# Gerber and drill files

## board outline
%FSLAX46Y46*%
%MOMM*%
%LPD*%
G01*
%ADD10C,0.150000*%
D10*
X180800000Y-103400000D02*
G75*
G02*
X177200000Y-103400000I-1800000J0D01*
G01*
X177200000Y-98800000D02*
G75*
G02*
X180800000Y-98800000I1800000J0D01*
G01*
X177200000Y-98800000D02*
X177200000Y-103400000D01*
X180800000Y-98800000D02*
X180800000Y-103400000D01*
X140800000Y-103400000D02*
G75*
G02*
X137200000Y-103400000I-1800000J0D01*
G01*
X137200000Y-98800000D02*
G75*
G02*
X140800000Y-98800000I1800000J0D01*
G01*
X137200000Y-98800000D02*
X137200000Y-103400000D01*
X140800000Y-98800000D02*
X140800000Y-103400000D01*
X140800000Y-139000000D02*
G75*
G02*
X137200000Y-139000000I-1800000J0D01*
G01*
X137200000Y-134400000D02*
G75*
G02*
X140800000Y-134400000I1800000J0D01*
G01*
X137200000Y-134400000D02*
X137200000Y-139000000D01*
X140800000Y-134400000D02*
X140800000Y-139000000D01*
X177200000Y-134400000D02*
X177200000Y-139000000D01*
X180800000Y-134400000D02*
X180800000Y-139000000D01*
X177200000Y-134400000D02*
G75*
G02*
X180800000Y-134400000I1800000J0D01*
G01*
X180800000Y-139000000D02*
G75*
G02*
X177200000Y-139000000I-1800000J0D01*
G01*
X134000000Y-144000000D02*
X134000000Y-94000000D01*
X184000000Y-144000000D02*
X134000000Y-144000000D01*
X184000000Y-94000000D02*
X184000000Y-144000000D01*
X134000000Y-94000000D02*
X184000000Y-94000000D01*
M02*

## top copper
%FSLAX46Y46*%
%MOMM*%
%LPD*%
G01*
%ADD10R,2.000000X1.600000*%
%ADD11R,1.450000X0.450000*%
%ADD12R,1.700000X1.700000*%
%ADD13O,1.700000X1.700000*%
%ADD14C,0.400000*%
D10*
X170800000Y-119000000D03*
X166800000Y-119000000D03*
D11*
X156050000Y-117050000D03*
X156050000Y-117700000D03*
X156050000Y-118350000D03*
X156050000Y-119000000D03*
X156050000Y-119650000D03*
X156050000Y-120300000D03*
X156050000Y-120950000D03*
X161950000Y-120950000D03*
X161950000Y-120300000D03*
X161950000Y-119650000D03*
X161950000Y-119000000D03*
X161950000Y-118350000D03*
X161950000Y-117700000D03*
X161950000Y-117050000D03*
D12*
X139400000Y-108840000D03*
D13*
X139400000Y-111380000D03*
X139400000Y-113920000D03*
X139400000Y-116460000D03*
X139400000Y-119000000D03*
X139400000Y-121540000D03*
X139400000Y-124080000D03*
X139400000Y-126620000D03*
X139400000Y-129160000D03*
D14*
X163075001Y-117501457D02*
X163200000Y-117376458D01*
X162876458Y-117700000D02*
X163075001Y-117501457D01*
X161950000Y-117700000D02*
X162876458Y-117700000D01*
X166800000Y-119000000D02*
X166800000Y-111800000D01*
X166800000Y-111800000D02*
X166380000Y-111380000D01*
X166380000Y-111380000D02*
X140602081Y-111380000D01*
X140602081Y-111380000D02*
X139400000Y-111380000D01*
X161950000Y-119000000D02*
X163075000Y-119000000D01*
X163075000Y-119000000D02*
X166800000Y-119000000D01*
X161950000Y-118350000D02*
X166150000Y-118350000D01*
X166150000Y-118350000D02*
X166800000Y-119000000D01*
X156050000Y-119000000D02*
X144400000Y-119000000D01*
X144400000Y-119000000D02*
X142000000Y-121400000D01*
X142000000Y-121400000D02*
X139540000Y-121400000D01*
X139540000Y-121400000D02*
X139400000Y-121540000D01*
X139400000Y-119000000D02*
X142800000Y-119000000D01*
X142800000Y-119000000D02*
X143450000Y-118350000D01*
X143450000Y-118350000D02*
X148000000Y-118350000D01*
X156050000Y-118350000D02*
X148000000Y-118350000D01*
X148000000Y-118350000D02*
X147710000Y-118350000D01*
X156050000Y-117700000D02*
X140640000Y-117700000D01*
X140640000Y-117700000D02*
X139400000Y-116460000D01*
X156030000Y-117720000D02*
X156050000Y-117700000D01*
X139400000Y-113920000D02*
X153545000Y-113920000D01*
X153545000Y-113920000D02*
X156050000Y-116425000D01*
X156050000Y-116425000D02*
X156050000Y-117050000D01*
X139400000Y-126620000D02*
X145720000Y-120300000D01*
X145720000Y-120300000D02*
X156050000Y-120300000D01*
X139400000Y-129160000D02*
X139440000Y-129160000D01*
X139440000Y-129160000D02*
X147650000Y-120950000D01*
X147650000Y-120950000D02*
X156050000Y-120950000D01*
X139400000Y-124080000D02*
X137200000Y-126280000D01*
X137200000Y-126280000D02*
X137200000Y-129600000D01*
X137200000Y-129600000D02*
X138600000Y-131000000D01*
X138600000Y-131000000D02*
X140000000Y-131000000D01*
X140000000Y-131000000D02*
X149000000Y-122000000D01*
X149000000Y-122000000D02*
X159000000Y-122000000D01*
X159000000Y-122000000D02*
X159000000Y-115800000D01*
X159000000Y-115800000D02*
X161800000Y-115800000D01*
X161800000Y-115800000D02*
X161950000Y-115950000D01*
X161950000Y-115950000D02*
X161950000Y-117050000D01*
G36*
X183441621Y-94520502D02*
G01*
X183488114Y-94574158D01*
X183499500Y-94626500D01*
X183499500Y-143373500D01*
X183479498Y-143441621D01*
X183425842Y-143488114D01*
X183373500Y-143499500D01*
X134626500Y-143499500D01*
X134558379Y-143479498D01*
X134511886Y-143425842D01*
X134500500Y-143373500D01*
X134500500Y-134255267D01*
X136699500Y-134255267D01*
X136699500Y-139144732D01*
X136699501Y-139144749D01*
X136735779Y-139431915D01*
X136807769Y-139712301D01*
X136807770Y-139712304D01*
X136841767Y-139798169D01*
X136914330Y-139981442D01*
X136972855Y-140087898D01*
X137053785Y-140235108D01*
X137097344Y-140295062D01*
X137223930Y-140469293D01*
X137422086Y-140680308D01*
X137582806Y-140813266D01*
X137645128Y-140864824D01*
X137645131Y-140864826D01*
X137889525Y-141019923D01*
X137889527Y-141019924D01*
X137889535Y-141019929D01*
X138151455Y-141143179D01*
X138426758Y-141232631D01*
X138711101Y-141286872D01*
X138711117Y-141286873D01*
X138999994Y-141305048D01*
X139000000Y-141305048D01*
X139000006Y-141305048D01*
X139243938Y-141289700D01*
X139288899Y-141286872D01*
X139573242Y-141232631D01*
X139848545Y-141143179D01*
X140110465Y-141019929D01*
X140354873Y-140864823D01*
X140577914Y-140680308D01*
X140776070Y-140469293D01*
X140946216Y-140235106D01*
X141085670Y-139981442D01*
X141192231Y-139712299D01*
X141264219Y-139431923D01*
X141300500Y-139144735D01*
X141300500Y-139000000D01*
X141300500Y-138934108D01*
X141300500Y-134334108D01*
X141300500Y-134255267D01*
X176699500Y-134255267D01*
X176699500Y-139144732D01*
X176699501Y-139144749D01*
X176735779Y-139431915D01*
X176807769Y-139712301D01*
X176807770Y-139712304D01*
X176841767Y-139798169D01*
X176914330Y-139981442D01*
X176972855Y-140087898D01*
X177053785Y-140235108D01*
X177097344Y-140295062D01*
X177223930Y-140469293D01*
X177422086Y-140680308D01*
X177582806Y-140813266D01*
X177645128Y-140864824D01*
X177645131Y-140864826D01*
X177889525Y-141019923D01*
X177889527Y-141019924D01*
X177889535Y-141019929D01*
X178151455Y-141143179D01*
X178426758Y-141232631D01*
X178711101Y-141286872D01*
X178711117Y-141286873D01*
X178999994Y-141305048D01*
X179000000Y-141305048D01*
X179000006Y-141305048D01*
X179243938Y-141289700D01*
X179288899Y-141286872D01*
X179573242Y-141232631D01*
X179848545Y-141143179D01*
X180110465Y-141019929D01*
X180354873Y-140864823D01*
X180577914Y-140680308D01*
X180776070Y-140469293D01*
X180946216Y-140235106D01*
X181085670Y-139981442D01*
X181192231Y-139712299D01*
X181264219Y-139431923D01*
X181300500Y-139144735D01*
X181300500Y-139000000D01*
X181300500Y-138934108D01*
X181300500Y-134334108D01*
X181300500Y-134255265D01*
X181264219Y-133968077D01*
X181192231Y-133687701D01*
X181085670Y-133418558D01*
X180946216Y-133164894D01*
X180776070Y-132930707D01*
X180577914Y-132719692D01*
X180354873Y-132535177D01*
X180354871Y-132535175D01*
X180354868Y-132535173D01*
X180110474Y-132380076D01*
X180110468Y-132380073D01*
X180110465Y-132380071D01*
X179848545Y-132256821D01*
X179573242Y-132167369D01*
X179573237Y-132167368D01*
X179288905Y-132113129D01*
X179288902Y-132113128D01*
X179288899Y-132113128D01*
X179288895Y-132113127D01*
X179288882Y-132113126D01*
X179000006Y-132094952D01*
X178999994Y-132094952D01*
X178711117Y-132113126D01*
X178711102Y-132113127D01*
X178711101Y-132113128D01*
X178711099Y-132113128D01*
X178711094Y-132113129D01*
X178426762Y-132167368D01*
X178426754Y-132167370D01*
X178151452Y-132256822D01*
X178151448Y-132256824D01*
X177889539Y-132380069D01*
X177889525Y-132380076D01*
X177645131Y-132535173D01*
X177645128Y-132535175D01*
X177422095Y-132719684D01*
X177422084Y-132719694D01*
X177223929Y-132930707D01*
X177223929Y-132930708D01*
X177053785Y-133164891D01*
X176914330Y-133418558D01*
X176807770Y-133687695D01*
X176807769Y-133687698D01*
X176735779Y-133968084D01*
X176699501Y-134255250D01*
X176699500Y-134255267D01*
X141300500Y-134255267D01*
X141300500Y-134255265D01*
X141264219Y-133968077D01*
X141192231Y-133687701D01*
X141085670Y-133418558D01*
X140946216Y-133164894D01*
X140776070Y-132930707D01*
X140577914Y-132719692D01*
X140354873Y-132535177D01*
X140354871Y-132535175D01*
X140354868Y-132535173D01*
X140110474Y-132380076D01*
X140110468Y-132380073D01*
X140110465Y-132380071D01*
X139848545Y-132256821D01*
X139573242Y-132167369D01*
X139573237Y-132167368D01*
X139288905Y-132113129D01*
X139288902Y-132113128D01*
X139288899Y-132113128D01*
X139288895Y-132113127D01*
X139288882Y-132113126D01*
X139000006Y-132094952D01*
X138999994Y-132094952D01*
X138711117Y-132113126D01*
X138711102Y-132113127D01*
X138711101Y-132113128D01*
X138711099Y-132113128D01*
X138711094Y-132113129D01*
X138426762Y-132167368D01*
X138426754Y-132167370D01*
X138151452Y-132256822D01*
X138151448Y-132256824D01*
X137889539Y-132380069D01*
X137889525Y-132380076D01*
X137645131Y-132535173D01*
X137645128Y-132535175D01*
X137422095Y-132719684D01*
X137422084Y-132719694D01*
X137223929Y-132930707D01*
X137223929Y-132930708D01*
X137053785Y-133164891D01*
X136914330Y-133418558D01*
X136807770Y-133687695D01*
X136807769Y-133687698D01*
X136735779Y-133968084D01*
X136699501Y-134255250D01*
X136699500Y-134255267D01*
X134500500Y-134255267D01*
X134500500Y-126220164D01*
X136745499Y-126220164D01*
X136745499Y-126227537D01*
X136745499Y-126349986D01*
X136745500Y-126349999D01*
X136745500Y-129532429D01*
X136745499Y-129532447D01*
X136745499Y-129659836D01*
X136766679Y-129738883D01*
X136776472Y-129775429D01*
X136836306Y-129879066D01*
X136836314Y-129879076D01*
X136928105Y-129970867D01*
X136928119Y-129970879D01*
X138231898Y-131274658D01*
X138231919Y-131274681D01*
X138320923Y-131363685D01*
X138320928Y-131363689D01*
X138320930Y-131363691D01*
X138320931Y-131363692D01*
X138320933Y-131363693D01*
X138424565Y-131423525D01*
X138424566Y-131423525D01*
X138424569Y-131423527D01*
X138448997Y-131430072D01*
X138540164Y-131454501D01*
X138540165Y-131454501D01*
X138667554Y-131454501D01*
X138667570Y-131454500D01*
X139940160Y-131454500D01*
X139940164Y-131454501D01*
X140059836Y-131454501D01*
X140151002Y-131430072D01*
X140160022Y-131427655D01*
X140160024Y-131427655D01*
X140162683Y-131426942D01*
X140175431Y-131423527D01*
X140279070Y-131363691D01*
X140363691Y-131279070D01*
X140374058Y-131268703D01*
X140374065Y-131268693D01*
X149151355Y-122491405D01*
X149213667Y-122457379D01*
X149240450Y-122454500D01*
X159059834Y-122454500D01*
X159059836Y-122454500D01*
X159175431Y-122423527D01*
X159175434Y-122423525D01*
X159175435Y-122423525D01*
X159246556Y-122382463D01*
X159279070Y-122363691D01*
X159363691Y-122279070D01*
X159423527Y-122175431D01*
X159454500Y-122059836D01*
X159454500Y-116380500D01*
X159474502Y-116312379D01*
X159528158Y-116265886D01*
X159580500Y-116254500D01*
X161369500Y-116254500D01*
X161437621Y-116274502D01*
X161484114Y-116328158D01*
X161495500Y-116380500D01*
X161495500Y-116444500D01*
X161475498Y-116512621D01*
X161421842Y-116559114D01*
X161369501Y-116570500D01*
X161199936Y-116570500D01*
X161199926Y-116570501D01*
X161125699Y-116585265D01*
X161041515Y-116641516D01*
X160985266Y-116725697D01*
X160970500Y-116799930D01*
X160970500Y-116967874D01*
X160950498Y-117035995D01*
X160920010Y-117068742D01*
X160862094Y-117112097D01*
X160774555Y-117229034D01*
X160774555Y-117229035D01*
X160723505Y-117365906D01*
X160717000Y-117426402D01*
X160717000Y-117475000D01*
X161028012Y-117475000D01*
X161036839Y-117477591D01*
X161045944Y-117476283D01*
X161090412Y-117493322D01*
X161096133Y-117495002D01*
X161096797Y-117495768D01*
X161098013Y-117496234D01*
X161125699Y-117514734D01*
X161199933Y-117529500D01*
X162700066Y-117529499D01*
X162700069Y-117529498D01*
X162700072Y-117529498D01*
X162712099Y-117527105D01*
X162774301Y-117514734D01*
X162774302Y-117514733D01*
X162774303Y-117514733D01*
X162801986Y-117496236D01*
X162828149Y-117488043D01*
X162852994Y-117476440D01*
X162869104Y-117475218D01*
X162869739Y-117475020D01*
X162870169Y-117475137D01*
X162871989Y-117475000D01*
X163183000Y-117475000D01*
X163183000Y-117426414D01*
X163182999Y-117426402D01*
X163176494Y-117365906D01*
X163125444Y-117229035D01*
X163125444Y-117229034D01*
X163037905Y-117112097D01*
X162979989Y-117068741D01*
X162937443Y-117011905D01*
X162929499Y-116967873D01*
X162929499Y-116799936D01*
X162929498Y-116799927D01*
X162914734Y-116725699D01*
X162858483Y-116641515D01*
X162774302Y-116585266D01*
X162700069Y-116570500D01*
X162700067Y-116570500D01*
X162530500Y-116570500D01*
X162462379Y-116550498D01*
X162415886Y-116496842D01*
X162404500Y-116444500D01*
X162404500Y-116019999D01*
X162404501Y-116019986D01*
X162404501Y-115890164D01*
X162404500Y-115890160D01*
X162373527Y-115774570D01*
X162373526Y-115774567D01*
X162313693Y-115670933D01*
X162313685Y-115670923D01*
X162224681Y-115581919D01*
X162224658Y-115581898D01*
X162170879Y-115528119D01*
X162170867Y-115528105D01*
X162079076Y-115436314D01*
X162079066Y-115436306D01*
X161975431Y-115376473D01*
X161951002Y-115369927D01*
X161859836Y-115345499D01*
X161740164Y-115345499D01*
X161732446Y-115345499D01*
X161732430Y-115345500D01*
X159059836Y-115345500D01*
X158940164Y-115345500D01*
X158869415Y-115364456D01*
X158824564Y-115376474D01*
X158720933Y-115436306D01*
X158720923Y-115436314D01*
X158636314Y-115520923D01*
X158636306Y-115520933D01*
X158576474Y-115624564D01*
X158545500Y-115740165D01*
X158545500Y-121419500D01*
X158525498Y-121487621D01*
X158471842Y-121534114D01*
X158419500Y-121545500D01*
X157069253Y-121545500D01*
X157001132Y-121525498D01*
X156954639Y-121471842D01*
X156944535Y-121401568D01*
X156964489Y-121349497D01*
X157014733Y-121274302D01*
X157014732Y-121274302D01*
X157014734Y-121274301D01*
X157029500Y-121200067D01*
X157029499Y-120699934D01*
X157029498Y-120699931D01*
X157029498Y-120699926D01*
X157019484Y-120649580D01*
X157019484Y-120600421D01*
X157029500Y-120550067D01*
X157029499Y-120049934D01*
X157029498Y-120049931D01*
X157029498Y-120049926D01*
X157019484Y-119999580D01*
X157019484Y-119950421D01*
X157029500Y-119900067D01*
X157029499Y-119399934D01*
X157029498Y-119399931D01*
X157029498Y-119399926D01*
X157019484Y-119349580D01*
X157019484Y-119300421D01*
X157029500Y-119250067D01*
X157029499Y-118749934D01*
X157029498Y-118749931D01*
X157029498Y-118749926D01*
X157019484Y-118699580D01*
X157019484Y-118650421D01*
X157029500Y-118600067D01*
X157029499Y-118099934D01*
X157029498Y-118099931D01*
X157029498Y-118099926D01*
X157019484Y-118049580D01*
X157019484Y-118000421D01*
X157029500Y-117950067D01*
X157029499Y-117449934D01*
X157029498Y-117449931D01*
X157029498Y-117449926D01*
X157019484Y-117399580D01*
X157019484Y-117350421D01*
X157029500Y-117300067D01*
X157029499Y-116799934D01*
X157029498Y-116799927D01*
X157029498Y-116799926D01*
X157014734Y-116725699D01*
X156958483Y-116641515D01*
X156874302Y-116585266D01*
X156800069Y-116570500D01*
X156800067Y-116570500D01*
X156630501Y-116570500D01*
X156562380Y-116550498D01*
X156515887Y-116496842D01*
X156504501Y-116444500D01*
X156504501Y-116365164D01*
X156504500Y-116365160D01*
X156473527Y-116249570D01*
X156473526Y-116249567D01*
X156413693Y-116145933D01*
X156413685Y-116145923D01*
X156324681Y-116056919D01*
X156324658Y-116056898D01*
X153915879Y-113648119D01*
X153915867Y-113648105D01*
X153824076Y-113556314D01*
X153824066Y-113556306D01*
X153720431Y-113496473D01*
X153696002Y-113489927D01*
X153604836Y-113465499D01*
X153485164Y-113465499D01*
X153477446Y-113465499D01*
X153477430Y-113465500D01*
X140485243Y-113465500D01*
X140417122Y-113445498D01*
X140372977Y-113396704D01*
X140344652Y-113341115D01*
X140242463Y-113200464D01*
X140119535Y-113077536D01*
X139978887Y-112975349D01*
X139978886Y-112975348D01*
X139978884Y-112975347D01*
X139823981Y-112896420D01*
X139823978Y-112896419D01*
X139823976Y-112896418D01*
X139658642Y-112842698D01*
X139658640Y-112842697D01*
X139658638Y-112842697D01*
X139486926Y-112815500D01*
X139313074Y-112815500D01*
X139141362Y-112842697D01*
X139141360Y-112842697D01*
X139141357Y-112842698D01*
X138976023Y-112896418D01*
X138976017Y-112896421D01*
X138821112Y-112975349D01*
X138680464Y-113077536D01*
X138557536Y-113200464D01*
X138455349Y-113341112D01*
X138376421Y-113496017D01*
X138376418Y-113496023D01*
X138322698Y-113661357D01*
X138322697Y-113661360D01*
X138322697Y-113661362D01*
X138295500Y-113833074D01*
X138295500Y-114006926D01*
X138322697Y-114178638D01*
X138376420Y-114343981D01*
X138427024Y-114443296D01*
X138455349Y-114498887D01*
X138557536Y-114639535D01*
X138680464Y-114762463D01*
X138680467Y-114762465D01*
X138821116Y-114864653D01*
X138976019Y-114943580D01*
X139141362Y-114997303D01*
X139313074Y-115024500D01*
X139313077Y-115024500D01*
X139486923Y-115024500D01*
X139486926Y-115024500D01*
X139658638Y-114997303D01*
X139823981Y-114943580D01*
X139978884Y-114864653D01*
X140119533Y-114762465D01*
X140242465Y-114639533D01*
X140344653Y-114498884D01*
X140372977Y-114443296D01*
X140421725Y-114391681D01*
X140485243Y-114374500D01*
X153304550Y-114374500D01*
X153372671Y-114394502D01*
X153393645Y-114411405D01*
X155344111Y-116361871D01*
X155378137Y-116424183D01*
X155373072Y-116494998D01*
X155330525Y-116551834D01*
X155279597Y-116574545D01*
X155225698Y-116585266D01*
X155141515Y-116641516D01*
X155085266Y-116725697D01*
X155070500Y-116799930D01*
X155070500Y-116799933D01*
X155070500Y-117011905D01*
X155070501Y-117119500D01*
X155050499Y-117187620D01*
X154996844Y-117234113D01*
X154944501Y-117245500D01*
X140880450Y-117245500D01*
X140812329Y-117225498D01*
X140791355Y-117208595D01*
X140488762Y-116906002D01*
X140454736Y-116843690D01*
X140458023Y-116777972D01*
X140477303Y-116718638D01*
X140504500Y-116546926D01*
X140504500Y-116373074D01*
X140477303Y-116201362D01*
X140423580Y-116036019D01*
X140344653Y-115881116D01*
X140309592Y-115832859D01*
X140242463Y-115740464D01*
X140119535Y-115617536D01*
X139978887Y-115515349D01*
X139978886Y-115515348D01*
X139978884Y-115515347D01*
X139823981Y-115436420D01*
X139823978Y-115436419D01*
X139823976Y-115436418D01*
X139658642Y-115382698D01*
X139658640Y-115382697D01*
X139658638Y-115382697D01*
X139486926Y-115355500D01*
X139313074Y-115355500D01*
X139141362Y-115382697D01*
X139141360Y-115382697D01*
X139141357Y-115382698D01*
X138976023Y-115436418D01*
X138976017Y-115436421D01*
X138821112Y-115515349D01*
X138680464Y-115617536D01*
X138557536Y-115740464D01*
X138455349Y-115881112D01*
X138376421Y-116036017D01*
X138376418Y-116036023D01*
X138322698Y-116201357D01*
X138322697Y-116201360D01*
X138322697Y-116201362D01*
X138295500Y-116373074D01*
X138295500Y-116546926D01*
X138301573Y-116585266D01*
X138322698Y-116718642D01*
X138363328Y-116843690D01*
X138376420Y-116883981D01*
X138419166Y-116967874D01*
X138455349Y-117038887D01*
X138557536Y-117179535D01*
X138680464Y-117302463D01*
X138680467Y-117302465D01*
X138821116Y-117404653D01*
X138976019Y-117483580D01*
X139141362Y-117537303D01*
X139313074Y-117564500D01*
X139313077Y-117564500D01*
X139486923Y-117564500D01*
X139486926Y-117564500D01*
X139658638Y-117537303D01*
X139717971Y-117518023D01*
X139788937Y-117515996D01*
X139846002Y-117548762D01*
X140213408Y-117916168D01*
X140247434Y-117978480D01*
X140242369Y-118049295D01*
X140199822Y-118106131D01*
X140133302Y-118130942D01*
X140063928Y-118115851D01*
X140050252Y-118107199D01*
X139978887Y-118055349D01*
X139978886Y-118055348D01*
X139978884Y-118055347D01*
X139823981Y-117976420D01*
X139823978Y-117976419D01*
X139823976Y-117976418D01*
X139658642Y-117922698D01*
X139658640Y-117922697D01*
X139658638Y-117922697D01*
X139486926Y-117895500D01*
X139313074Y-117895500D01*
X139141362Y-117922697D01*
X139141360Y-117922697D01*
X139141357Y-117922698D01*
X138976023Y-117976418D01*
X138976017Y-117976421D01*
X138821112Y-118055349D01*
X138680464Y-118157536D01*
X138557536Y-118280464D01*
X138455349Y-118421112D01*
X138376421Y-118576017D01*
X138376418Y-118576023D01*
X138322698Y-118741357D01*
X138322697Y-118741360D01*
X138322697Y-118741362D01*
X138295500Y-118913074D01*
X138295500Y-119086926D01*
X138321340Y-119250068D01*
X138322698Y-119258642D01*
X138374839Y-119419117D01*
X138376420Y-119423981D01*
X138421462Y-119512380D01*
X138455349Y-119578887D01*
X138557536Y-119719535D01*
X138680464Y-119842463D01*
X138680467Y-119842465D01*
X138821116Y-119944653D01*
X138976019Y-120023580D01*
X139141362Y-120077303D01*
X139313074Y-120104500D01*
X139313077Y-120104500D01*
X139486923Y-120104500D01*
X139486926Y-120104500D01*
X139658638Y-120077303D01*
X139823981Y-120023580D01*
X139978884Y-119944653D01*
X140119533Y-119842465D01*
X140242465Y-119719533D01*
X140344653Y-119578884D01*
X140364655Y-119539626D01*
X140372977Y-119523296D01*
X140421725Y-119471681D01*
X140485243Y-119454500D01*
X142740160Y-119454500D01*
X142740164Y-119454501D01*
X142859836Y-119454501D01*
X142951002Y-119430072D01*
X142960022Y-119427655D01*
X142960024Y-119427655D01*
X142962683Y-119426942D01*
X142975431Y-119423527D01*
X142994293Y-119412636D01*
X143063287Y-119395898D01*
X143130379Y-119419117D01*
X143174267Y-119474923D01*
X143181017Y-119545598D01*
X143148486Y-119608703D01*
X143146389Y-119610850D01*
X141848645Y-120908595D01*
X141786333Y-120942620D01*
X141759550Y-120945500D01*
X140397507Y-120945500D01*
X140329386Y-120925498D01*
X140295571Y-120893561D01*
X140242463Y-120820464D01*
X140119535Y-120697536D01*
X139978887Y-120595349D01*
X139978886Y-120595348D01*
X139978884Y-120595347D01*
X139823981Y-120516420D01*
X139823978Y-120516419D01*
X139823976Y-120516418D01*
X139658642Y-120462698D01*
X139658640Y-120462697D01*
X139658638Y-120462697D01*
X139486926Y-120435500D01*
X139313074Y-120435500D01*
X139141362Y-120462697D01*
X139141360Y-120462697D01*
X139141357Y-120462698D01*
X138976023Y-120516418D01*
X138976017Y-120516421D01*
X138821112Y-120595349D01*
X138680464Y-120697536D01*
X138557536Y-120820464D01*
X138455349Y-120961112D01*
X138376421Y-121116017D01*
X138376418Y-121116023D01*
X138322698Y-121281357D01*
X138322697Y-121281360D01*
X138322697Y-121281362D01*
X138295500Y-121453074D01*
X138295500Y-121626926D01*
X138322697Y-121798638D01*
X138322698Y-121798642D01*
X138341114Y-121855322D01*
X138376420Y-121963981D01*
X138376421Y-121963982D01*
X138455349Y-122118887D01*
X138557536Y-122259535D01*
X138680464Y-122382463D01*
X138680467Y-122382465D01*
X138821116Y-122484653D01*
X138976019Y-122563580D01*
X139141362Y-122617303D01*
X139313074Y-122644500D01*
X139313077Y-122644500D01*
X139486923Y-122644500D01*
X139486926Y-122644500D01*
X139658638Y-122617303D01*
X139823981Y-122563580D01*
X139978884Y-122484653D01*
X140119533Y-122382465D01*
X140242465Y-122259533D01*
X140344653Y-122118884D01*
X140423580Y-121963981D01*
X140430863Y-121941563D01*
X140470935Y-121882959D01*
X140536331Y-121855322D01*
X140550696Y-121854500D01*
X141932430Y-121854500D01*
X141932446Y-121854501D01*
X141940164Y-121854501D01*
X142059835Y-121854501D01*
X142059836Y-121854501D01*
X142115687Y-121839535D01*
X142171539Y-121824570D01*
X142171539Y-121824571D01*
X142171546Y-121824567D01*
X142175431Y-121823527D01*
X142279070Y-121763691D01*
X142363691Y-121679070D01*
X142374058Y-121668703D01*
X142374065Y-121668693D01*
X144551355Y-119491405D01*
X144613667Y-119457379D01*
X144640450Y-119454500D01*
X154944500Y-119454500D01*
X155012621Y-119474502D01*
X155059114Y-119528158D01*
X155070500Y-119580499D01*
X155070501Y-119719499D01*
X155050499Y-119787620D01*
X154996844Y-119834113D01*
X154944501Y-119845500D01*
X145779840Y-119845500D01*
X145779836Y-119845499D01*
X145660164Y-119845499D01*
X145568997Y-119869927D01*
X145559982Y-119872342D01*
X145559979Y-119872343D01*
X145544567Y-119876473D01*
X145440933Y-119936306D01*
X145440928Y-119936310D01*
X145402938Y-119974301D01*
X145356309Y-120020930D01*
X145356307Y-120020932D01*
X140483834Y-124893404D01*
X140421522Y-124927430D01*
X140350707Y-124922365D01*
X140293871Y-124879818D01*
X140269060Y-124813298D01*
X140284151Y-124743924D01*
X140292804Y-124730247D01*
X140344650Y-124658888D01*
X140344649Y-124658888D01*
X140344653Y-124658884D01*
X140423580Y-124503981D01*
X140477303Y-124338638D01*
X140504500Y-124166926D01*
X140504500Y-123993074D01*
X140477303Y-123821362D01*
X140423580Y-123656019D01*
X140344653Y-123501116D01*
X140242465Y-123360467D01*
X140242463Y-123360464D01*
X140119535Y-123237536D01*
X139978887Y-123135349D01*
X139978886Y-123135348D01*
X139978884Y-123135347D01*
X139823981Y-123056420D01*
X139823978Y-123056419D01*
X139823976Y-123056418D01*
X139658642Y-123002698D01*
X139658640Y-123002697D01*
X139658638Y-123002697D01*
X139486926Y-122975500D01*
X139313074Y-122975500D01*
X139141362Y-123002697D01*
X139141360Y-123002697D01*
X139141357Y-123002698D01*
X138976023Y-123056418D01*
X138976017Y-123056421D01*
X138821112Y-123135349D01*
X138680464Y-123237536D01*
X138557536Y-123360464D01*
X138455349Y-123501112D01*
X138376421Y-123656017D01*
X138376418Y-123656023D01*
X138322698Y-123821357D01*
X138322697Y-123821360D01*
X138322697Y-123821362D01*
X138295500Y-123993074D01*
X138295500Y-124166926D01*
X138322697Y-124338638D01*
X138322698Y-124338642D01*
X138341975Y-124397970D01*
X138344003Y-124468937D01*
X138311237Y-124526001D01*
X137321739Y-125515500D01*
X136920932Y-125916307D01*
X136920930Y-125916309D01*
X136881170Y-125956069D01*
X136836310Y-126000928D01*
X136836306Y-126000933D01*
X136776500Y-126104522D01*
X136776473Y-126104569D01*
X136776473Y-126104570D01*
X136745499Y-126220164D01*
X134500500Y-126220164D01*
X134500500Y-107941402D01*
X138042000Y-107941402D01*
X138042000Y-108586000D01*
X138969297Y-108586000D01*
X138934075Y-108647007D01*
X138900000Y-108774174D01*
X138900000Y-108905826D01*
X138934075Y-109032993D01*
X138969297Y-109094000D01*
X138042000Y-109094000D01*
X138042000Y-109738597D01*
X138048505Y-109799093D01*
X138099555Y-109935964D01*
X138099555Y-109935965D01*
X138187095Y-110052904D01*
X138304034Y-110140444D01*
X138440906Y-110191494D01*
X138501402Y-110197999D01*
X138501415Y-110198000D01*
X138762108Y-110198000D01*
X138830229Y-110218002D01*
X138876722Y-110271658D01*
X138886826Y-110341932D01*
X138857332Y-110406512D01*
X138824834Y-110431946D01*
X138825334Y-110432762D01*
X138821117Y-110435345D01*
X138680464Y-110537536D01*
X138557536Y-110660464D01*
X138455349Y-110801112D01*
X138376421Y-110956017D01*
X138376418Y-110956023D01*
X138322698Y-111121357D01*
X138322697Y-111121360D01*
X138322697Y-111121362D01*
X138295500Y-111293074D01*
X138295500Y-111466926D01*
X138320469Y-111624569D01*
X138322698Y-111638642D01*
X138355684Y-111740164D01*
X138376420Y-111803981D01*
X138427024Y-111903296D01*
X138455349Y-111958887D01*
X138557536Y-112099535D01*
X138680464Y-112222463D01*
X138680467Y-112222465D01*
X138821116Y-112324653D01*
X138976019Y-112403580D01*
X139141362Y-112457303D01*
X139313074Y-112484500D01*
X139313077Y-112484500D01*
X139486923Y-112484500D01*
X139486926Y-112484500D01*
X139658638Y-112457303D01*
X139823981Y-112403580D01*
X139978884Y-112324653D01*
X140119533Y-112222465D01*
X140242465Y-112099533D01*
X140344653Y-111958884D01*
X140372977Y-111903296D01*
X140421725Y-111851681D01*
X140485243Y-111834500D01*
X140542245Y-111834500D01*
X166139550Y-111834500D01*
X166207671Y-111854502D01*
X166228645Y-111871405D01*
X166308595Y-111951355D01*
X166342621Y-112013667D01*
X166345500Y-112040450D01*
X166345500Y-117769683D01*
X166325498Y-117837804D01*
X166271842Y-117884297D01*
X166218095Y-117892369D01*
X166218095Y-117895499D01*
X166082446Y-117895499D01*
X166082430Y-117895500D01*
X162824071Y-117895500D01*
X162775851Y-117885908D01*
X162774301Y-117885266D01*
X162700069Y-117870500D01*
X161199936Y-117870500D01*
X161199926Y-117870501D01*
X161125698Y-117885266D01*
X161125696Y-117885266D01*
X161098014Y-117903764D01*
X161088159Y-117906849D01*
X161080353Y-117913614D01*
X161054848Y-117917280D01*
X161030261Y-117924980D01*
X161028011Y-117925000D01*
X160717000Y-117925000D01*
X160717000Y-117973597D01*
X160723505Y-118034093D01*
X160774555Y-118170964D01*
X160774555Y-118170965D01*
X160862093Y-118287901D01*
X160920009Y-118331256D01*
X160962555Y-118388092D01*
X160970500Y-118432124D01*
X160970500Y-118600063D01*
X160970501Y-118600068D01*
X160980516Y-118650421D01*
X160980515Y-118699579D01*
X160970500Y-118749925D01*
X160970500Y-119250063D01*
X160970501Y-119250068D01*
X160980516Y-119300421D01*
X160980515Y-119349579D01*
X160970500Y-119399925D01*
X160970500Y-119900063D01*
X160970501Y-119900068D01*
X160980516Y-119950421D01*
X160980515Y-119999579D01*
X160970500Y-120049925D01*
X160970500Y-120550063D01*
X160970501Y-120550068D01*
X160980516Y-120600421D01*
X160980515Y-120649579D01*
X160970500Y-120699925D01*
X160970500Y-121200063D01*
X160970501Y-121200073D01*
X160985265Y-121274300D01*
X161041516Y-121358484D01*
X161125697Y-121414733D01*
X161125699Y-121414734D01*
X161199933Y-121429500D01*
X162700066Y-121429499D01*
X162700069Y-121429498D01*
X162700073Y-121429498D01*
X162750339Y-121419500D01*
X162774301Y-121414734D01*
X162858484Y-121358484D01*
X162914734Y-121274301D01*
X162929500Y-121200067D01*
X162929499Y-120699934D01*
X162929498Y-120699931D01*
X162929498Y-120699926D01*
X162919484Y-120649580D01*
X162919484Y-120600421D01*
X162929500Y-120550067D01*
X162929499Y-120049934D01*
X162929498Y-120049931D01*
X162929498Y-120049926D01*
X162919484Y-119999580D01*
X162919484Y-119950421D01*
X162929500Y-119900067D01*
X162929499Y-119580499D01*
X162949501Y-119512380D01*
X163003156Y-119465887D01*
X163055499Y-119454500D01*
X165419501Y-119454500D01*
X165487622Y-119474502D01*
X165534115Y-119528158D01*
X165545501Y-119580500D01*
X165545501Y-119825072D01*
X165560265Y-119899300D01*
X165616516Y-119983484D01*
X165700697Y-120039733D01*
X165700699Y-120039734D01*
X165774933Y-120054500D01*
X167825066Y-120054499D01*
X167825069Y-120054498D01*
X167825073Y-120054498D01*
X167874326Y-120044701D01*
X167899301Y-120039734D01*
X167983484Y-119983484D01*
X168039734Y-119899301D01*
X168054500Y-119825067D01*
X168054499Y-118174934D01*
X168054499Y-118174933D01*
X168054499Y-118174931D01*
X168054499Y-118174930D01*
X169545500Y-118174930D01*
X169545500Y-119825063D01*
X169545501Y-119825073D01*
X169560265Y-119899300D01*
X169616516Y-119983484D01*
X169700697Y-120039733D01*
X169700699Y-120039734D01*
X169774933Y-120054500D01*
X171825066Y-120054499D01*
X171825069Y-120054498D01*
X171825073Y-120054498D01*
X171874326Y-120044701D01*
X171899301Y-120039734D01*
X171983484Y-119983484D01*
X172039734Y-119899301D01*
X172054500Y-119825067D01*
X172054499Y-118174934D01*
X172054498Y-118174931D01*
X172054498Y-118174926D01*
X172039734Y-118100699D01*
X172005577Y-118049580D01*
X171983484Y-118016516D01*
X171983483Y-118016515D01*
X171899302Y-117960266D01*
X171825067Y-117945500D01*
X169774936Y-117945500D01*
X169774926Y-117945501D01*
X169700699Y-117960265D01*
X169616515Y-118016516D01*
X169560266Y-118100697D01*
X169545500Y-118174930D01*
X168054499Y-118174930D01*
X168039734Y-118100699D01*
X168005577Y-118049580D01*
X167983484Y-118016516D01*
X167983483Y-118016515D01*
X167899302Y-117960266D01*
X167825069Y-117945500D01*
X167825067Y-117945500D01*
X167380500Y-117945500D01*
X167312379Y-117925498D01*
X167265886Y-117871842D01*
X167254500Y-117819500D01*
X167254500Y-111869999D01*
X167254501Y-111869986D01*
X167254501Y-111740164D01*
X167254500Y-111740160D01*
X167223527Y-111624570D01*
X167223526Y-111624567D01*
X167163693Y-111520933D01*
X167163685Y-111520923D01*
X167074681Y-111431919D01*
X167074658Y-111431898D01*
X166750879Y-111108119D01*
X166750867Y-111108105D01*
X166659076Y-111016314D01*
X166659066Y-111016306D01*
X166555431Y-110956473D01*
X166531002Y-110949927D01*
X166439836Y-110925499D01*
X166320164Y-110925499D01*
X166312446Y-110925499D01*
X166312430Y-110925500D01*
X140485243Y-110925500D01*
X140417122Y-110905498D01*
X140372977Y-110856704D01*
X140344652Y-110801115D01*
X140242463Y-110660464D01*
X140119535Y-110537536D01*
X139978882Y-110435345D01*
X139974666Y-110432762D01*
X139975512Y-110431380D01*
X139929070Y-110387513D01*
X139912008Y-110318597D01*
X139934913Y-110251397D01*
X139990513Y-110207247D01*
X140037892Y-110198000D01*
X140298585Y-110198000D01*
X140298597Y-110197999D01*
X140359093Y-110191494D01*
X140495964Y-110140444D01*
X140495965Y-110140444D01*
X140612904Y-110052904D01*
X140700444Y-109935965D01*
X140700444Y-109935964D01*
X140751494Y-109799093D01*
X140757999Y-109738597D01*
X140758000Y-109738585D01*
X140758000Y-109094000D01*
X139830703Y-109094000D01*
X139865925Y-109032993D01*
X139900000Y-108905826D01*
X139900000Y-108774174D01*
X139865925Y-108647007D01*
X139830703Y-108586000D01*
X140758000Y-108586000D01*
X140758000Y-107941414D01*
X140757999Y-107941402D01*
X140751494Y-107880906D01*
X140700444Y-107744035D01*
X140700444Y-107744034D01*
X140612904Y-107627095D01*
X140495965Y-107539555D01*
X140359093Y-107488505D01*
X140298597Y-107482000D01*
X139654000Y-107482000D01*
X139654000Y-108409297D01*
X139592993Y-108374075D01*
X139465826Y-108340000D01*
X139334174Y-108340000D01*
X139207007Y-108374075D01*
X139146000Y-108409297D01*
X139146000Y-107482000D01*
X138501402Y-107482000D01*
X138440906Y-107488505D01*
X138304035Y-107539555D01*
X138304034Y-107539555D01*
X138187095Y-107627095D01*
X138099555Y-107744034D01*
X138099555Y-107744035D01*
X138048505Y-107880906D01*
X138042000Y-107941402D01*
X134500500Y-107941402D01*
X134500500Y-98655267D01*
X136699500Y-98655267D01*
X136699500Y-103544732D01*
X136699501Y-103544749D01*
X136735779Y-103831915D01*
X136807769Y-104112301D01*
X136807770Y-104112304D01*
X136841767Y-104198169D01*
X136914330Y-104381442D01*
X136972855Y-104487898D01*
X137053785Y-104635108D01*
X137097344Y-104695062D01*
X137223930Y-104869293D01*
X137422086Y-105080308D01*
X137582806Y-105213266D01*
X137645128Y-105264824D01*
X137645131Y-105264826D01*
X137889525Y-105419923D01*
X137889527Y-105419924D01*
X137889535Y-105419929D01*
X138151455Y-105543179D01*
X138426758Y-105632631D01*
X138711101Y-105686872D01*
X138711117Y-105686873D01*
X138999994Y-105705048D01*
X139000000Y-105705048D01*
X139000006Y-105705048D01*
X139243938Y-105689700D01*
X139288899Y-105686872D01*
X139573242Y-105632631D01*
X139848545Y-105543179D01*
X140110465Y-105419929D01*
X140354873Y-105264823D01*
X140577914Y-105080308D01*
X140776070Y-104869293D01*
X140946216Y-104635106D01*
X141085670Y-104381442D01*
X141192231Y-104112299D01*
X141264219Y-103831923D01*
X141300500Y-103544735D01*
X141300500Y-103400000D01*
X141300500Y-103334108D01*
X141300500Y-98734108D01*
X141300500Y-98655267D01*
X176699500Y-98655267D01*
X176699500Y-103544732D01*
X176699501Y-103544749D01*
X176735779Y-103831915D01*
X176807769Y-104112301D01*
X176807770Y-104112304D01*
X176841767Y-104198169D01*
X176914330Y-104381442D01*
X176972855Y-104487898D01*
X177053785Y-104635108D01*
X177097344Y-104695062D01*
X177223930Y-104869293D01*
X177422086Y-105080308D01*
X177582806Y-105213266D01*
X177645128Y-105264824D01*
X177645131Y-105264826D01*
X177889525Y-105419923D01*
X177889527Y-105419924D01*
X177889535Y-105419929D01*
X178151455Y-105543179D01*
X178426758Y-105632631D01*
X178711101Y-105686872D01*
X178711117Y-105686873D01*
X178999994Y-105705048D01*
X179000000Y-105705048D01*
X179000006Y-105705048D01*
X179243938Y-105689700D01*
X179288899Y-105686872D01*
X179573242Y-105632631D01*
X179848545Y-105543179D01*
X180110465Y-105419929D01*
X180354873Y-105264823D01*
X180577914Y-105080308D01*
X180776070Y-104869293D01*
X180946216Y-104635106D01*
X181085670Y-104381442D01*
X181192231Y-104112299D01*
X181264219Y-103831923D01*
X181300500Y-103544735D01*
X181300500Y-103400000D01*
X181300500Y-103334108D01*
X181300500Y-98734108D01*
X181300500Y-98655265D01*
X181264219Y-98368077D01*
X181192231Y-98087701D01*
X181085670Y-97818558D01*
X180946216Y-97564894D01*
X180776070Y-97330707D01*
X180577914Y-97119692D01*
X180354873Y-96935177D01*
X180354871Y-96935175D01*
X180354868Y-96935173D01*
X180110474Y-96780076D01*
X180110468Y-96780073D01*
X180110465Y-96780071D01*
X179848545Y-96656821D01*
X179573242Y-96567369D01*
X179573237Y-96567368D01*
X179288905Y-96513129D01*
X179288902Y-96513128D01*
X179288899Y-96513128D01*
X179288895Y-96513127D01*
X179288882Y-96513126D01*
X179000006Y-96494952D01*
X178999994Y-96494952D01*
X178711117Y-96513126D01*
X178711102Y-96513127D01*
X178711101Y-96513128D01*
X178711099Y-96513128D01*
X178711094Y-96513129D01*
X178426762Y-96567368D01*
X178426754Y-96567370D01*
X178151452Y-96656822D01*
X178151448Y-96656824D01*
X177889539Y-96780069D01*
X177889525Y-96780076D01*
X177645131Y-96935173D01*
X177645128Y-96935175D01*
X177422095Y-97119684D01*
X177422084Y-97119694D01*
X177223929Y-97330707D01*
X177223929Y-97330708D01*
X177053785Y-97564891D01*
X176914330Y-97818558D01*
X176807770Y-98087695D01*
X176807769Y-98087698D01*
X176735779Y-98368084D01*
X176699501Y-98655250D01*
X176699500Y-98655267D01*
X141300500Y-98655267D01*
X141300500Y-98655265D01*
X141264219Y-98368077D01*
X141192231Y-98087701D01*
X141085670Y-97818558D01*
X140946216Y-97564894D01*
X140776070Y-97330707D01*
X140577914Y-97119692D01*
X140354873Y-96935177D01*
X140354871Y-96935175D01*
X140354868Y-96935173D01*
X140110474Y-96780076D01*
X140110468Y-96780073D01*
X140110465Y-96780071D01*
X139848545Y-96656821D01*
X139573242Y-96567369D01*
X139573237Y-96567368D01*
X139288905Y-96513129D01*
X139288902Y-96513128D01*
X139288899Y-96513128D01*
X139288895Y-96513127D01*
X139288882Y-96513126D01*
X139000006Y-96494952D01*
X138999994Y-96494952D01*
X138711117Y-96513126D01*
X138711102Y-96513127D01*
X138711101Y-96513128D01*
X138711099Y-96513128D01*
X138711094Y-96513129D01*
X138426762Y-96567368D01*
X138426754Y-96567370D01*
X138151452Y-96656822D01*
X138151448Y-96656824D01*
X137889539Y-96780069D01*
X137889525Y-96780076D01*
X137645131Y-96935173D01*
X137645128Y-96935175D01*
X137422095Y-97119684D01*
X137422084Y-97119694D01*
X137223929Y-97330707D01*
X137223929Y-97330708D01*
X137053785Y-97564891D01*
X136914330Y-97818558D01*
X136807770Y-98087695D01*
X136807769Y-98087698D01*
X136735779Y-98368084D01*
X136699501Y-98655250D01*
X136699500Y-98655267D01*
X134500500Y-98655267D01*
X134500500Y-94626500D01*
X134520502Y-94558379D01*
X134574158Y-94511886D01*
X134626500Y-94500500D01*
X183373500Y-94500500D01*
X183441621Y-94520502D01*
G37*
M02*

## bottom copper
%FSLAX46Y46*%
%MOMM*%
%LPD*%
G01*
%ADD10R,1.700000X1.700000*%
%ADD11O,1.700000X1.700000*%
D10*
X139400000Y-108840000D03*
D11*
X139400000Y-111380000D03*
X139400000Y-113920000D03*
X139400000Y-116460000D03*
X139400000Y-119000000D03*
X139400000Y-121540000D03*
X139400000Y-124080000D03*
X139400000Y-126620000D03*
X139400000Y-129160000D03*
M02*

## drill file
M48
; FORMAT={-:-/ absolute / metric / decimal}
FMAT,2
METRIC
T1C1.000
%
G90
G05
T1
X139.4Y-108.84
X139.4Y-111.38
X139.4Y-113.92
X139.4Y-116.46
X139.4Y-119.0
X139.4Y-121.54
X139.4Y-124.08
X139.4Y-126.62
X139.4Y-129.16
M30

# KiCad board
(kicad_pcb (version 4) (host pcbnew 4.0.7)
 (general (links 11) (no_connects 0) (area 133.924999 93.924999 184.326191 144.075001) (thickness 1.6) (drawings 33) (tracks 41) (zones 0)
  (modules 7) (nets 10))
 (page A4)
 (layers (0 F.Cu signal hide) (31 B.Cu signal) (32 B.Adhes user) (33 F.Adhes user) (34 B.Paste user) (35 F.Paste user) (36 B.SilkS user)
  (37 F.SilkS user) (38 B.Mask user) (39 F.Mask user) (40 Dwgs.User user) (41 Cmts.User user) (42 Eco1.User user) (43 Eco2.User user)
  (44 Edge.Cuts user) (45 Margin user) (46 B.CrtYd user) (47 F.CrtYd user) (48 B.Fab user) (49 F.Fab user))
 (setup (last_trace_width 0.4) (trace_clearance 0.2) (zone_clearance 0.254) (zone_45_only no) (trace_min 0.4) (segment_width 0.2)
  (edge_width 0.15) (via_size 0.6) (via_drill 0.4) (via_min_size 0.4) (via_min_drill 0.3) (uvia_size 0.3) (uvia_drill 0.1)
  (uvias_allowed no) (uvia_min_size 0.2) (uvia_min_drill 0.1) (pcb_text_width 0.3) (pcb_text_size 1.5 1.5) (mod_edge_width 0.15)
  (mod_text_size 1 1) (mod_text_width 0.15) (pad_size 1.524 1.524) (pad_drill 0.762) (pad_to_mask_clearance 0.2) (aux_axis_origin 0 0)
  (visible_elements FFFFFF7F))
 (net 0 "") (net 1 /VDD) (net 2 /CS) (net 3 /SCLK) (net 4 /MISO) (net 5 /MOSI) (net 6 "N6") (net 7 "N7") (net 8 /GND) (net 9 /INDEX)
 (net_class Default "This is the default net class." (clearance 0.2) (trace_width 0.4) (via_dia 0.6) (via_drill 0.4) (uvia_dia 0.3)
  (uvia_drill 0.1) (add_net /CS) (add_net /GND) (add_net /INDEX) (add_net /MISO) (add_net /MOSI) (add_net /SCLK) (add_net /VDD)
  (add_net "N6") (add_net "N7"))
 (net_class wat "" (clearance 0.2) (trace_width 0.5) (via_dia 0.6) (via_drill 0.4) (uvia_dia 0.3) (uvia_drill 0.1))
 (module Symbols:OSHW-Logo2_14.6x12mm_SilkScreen (layer B.Cu) (at 169.4 133.2 180)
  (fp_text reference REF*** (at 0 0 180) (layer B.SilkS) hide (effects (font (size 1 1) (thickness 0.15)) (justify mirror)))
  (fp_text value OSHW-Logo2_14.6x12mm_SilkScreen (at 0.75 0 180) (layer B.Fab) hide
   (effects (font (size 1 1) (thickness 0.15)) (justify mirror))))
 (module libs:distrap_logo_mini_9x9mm (layer B.Cu) (at 168.5 103 180)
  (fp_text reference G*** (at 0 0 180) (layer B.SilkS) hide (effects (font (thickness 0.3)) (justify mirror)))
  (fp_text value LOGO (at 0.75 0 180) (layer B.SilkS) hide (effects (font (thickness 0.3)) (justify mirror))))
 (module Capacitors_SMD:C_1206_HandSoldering (layer F.Cu) (at 168.8 119 180)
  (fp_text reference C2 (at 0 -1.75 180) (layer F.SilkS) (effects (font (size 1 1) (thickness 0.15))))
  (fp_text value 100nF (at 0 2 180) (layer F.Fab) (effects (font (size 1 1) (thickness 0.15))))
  (pad 1 smd rect (at -2 0 180) (size 2 1.6) (layers F.Cu F.Paste F.Mask))
  (pad 2 smd rect (at 2 0 180) (size 2 1.6) (layers F.Cu F.Paste F.Mask) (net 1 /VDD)))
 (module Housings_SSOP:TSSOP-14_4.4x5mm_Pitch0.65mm (layer F.Cu) (at 159 119)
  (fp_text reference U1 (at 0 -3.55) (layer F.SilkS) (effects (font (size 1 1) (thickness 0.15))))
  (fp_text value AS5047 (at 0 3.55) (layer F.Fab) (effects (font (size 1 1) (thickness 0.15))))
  (pad 1 smd rect (at -2.95 -1.95) (size 1.45 0.45) (layers F.Cu F.Paste F.Mask) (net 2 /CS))
  (pad 2 smd rect (at -2.95 -1.3) (size 1.45 0.45) (layers F.Cu F.Paste F.Mask) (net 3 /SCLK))
  (pad 3 smd rect (at -2.95 -0.65) (size 1.45 0.45) (layers F.Cu F.Paste F.Mask) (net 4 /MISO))
  (pad 4 smd rect (at -2.95 0) (size 1.45 0.45) (layers F.Cu F.Paste F.Mask) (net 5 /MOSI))
  (pad 5 smd rect (at -2.95 0.65) (size 1.45 0.45) (layers F.Cu F.Paste F.Mask))
  (pad 6 smd rect (at -2.95 1.3) (size 1.45 0.45) (layers F.Cu F.Paste F.Mask) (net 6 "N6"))
  (pad 7 smd rect (at -2.95 1.95) (size 1.45 0.45) (layers F.Cu F.Paste F.Mask) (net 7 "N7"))
  (pad 8 smd rect (at 2.95 1.95) (size 1.45 0.45) (layers F.Cu F.Paste F.Mask))
  (pad 9 smd rect (at 2.95 1.3) (size 1.45 0.45) (layers F.Cu F.Paste F.Mask))
  (pad 10 smd rect (at 2.95 0.65) (size 1.45 0.45) (layers F.Cu F.Paste F.Mask))
  (pad 11 smd rect (at 2.95 0) (size 1.45 0.45) (layers F.Cu F.Paste F.Mask) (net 1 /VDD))
  (pad 12 smd rect (at 2.95 -0.65) (size 1.45 0.45) (layers F.Cu F.Paste F.Mask) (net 1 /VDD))
  (pad 13 smd rect (at 2.95 -1.3) (size 1.45 0.45) (layers F.Cu F.Paste F.Mask) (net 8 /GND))
  (pad 14 smd rect (at 2.95 -1.95) (size 1.45 0.45) (layers F.Cu F.Paste F.Mask) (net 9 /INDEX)))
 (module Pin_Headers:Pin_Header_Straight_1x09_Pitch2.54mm (layer B.Cu) (at 139.4 108.84 180)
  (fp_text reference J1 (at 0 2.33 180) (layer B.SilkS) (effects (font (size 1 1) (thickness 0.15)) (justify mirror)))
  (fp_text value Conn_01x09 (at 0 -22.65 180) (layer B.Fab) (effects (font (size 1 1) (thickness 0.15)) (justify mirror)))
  (pad 1 thru_hole rect (at 0 0 180) (size 1.7 1.7) (drill 1) (layers *.Cu *.Mask) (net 8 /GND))
  (pad 2 thru_hole oval (at 0 -2.54 180) (size 1.7 1.7) (drill 1) (layers *.Cu *.Mask) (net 1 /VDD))
  (pad 3 thru_hole oval (at 0 -5.08 180) (size 1.7 1.7) (drill 1) (layers *.Cu *.Mask) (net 2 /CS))
  (pad 4 thru_hole oval (at 0 -7.62 180) (size 1.7 1.7) (drill 1) (layers *.Cu *.Mask) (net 3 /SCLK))
  (pad 5 thru_hole oval (at 0 -10.16 180) (size 1.7 1.7) (drill 1) (layers *.Cu *.Mask) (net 4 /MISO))
  (pad 6 thru_hole oval (at 0 -12.7 180) (size 1.7 1.7) (drill 1) (layers *.Cu *.Mask) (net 5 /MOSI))
  (pad 7 thru_hole oval (at 0 -15.24 180) (size 1.7 1.7) (drill 1) (layers *.Cu *.Mask) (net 9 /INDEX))
  (pad 8 thru_hole oval (at 0 -17.78 180) (size 1.7 1.7) (drill 1) (layers *.Cu *.Mask) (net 6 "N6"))
  (pad 9 thru_hole oval (at 0 -20.32 180) (size 1.7 1.7) (drill 1) (layers *.Cu *.Mask) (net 7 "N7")))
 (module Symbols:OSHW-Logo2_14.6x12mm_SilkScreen (layer F.Cu) (at 169.4 133.2)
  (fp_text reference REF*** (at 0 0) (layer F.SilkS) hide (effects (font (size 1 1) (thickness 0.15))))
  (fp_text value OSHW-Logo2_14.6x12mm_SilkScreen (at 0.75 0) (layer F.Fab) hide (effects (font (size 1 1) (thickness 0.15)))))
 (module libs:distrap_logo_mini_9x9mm (layer F.Cu) (at 168.5 103)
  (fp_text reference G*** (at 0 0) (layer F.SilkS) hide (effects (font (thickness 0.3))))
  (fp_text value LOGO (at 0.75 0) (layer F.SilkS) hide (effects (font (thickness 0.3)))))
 (gr_arc (start 179 103.4) (end 180.8 103.4) (angle 180) (layer Edge.Cuts) (width 0.15))
 (gr_arc (start 179 98.8) (end 177.2 98.8) (angle 180) (layer Edge.Cuts) (width 0.15))
 (gr_line (start 177.2 98.8) (end 177.2 103.4) (layer Edge.Cuts) (width 0.15))
 (gr_line (start 180.8 98.8) (end 180.8 103.4) (layer Edge.Cuts) (width 0.15))
 (gr_arc (start 139 103.4) (end 140.8 103.4) (angle 180) (layer Edge.Cuts) (width 0.15))
 (gr_arc (start 139 98.8) (end 137.2 98.8) (angle 180) (layer Edge.Cuts) (width 0.15))
 (gr_line (start 137.2 98.8) (end 137.2 103.4) (layer Edge.Cuts) (width 0.15))
 (gr_line (start 140.8 98.8) (end 140.8 103.4) (layer Edge.Cuts) (width 0.15))
 (gr_arc (start 139 139) (end 140.8 139) (angle 180) (layer Edge.Cuts) (width 0.15))
 (gr_arc (start 139 134.4) (end 137.2 134.4) (angle 180) (layer Edge.Cuts) (width 0.15))
 (gr_line (start 137.2 134.4) (end 137.2 139) (layer Edge.Cuts) (width 0.15))
 (gr_line (start 140.8 134.4) (end 140.8 139) (layer Edge.Cuts) (width 0.15))
 (gr_line (start 177.2 134.4) (end 177.2 139) (layer Edge.Cuts) (width 0.15))
 (gr_line (start 180.8 134.4) (end 180.8 139) (layer Edge.Cuts) (width 0.15))
 (gr_arc (start 179 134.4) (end 177.2 134.4) (angle 180) (layer Edge.Cuts) (width 0.15))
 (gr_arc (start 179 139) (end 180.8 139) (angle 180) (layer Edge.Cuts) (width 0.15))
 (gr_line (start 134 144) (end 134 94) (layer Edge.Cuts) (width 0.15))
 (gr_line (start 184 144) (end 134 144) (layer Edge.Cuts) (width 0.15))
 (gr_line (start 184 94) (end 184 144) (layer Edge.Cuts) (width 0.15))
 (gr_line (start 134 94) (end 184 94) (layer Edge.Cuts) (width 0.15))
 (segment (start 163.075001 117.501457) (end 163.2 117.376458) (width 0.4) (layer F.Cu) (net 8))
 (segment (start 162.876458 117.7) (end 163.075001 117.501457) (width 0.4) (layer F.Cu) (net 8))
 (segment (start 161.95 117.7) (end 162.876458 117.7) (width 0.4) (layer F.Cu) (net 8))
 (segment (start 166.8 119) (end 166.8 111.8) (width 0.4) (layer F.Cu) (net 1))
 (segment (start 166.8 111.8) (end 166.38 111.38) (width 0.4) (layer F.Cu) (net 1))
 (segment (start 166.38 111.38) (end 140.602081 111.38) (width 0.4) (layer F.Cu) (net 1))
 (segment (start 140.602081 111.38) (end 139.4 111.38) (width 0.4) (layer F.Cu) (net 1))
 (segment (start 161.95 119) (end 163.075 119) (width 0.4) (layer F.Cu) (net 1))
 (segment (start 163.075 119) (end 166.8 119) (width 0.4) (layer F.Cu) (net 1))
 (segment (start 161.95 118.35) (end 166.15 118.35) (width 0.4) (layer F.Cu) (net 1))
 (segment (start 166.15 118.35) (end 166.8 119) (width 0.4) (layer F.Cu) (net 1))
 (segment (start 156.05 119) (end 144.4 119) (width 0.4) (layer F.Cu) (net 5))
 (segment (start 144.4 119) (end 142 121.4) (width 0.4) (layer F.Cu) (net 5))
 (segment (start 142 121.4) (end 139.54 121.4) (width 0.4) (layer F.Cu) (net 5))
 (segment (start 139.54 121.4) (end 139.4 121.54) (width 0.4) (layer F.Cu) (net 5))
 (segment (start 139.4 119) (end 142.8 119) (width 0.4) (layer F.Cu) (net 4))
 (segment (start 142.8 119) (end 143.45 118.35) (width 0.4) (layer F.Cu) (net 4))
 (segment (start 143.45 118.35) (end 148 118.35) (width 0.4) (layer F.Cu) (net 4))
 (segment (start 156.05 118.35) (end 148 118.35) (width 0.4) (layer F.Cu) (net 4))
 (segment (start 148 118.35) (end 147.71 118.35) (width 0.4) (layer F.Cu) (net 4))
 (segment (start 156.05 117.7) (end 140.64 117.7) (width 0.4) (layer F.Cu) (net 3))
 (segment (start 140.64 117.7) (end 139.4 116.46) (width 0.4) (layer F.Cu) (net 3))
 (segment (start 156.03 117.72) (end 156.05 117.7) (width 0.4) (layer F.Cu) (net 3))
 (segment (start 139.4 113.92) (end 153.545 113.92) (width 0.4) (layer F.Cu) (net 2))
 (segment (start 153.545 113.92) (end 156.05 116.425) (width 0.4) (layer F.Cu) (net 2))
 (segment (start 156.05 116.425) (end 156.05 117.05) (width 0.4) (layer F.Cu) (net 2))
 (segment (start 139.4 126.62) (end 145.72 120.3) (width 0.4) (layer F.Cu) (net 6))
 (segment (start 145.72 120.3) (end 156.05 120.3) (width 0.4) (layer F.Cu) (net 6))
 (segment (start 139.4 129.16) (end 139.44 129.16) (width 0.4) (layer F.Cu) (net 7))
 (segment (start 139.44 129.16) (end 147.65 120.95) (width 0.4) (layer F.Cu) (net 7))
 (segment (start 147.65 120.95) (end 156.05 120.95) (width 0.4) (layer F.Cu) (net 7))
 (segment (start 139.4 124.08) (end 137.2 126.28) (width 0.4) (layer F.Cu) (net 9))
 (segment (start 137.2 126.28) (end 137.2 129.6) (width 0.4) (layer F.Cu) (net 9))
 (segment (start 137.2 129.6) (end 138.6 131) (width 0.4) (layer F.Cu) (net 9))
 (segment (start 138.6 131) (end 140 131) (width 0.4) (layer F.Cu) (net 9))
 (segment (start 140 131) (end 149 122) (width 0.4) (layer F.Cu) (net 9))
 (segment (start 149 122) (end 159 122) (width 0.4) (layer F.Cu) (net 9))
 (segment (start 159 122) (end 159 115.8) (width 0.4) (layer F.Cu) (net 9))
 (segment (start 159 115.8) (end 161.8 115.8) (width 0.4) (layer F.Cu) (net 9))
 (segment (start 161.8 115.8) (end 161.95 115.95) (width 0.4) (layer F.Cu) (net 9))
 (segment (start 161.95 115.95) (end 161.95 117.05) (width 0.4) (layer F.Cu) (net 9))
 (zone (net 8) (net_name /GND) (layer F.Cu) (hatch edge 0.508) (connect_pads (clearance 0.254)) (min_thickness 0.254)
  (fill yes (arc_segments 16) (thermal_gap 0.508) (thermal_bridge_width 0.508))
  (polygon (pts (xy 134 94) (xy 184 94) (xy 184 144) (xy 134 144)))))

